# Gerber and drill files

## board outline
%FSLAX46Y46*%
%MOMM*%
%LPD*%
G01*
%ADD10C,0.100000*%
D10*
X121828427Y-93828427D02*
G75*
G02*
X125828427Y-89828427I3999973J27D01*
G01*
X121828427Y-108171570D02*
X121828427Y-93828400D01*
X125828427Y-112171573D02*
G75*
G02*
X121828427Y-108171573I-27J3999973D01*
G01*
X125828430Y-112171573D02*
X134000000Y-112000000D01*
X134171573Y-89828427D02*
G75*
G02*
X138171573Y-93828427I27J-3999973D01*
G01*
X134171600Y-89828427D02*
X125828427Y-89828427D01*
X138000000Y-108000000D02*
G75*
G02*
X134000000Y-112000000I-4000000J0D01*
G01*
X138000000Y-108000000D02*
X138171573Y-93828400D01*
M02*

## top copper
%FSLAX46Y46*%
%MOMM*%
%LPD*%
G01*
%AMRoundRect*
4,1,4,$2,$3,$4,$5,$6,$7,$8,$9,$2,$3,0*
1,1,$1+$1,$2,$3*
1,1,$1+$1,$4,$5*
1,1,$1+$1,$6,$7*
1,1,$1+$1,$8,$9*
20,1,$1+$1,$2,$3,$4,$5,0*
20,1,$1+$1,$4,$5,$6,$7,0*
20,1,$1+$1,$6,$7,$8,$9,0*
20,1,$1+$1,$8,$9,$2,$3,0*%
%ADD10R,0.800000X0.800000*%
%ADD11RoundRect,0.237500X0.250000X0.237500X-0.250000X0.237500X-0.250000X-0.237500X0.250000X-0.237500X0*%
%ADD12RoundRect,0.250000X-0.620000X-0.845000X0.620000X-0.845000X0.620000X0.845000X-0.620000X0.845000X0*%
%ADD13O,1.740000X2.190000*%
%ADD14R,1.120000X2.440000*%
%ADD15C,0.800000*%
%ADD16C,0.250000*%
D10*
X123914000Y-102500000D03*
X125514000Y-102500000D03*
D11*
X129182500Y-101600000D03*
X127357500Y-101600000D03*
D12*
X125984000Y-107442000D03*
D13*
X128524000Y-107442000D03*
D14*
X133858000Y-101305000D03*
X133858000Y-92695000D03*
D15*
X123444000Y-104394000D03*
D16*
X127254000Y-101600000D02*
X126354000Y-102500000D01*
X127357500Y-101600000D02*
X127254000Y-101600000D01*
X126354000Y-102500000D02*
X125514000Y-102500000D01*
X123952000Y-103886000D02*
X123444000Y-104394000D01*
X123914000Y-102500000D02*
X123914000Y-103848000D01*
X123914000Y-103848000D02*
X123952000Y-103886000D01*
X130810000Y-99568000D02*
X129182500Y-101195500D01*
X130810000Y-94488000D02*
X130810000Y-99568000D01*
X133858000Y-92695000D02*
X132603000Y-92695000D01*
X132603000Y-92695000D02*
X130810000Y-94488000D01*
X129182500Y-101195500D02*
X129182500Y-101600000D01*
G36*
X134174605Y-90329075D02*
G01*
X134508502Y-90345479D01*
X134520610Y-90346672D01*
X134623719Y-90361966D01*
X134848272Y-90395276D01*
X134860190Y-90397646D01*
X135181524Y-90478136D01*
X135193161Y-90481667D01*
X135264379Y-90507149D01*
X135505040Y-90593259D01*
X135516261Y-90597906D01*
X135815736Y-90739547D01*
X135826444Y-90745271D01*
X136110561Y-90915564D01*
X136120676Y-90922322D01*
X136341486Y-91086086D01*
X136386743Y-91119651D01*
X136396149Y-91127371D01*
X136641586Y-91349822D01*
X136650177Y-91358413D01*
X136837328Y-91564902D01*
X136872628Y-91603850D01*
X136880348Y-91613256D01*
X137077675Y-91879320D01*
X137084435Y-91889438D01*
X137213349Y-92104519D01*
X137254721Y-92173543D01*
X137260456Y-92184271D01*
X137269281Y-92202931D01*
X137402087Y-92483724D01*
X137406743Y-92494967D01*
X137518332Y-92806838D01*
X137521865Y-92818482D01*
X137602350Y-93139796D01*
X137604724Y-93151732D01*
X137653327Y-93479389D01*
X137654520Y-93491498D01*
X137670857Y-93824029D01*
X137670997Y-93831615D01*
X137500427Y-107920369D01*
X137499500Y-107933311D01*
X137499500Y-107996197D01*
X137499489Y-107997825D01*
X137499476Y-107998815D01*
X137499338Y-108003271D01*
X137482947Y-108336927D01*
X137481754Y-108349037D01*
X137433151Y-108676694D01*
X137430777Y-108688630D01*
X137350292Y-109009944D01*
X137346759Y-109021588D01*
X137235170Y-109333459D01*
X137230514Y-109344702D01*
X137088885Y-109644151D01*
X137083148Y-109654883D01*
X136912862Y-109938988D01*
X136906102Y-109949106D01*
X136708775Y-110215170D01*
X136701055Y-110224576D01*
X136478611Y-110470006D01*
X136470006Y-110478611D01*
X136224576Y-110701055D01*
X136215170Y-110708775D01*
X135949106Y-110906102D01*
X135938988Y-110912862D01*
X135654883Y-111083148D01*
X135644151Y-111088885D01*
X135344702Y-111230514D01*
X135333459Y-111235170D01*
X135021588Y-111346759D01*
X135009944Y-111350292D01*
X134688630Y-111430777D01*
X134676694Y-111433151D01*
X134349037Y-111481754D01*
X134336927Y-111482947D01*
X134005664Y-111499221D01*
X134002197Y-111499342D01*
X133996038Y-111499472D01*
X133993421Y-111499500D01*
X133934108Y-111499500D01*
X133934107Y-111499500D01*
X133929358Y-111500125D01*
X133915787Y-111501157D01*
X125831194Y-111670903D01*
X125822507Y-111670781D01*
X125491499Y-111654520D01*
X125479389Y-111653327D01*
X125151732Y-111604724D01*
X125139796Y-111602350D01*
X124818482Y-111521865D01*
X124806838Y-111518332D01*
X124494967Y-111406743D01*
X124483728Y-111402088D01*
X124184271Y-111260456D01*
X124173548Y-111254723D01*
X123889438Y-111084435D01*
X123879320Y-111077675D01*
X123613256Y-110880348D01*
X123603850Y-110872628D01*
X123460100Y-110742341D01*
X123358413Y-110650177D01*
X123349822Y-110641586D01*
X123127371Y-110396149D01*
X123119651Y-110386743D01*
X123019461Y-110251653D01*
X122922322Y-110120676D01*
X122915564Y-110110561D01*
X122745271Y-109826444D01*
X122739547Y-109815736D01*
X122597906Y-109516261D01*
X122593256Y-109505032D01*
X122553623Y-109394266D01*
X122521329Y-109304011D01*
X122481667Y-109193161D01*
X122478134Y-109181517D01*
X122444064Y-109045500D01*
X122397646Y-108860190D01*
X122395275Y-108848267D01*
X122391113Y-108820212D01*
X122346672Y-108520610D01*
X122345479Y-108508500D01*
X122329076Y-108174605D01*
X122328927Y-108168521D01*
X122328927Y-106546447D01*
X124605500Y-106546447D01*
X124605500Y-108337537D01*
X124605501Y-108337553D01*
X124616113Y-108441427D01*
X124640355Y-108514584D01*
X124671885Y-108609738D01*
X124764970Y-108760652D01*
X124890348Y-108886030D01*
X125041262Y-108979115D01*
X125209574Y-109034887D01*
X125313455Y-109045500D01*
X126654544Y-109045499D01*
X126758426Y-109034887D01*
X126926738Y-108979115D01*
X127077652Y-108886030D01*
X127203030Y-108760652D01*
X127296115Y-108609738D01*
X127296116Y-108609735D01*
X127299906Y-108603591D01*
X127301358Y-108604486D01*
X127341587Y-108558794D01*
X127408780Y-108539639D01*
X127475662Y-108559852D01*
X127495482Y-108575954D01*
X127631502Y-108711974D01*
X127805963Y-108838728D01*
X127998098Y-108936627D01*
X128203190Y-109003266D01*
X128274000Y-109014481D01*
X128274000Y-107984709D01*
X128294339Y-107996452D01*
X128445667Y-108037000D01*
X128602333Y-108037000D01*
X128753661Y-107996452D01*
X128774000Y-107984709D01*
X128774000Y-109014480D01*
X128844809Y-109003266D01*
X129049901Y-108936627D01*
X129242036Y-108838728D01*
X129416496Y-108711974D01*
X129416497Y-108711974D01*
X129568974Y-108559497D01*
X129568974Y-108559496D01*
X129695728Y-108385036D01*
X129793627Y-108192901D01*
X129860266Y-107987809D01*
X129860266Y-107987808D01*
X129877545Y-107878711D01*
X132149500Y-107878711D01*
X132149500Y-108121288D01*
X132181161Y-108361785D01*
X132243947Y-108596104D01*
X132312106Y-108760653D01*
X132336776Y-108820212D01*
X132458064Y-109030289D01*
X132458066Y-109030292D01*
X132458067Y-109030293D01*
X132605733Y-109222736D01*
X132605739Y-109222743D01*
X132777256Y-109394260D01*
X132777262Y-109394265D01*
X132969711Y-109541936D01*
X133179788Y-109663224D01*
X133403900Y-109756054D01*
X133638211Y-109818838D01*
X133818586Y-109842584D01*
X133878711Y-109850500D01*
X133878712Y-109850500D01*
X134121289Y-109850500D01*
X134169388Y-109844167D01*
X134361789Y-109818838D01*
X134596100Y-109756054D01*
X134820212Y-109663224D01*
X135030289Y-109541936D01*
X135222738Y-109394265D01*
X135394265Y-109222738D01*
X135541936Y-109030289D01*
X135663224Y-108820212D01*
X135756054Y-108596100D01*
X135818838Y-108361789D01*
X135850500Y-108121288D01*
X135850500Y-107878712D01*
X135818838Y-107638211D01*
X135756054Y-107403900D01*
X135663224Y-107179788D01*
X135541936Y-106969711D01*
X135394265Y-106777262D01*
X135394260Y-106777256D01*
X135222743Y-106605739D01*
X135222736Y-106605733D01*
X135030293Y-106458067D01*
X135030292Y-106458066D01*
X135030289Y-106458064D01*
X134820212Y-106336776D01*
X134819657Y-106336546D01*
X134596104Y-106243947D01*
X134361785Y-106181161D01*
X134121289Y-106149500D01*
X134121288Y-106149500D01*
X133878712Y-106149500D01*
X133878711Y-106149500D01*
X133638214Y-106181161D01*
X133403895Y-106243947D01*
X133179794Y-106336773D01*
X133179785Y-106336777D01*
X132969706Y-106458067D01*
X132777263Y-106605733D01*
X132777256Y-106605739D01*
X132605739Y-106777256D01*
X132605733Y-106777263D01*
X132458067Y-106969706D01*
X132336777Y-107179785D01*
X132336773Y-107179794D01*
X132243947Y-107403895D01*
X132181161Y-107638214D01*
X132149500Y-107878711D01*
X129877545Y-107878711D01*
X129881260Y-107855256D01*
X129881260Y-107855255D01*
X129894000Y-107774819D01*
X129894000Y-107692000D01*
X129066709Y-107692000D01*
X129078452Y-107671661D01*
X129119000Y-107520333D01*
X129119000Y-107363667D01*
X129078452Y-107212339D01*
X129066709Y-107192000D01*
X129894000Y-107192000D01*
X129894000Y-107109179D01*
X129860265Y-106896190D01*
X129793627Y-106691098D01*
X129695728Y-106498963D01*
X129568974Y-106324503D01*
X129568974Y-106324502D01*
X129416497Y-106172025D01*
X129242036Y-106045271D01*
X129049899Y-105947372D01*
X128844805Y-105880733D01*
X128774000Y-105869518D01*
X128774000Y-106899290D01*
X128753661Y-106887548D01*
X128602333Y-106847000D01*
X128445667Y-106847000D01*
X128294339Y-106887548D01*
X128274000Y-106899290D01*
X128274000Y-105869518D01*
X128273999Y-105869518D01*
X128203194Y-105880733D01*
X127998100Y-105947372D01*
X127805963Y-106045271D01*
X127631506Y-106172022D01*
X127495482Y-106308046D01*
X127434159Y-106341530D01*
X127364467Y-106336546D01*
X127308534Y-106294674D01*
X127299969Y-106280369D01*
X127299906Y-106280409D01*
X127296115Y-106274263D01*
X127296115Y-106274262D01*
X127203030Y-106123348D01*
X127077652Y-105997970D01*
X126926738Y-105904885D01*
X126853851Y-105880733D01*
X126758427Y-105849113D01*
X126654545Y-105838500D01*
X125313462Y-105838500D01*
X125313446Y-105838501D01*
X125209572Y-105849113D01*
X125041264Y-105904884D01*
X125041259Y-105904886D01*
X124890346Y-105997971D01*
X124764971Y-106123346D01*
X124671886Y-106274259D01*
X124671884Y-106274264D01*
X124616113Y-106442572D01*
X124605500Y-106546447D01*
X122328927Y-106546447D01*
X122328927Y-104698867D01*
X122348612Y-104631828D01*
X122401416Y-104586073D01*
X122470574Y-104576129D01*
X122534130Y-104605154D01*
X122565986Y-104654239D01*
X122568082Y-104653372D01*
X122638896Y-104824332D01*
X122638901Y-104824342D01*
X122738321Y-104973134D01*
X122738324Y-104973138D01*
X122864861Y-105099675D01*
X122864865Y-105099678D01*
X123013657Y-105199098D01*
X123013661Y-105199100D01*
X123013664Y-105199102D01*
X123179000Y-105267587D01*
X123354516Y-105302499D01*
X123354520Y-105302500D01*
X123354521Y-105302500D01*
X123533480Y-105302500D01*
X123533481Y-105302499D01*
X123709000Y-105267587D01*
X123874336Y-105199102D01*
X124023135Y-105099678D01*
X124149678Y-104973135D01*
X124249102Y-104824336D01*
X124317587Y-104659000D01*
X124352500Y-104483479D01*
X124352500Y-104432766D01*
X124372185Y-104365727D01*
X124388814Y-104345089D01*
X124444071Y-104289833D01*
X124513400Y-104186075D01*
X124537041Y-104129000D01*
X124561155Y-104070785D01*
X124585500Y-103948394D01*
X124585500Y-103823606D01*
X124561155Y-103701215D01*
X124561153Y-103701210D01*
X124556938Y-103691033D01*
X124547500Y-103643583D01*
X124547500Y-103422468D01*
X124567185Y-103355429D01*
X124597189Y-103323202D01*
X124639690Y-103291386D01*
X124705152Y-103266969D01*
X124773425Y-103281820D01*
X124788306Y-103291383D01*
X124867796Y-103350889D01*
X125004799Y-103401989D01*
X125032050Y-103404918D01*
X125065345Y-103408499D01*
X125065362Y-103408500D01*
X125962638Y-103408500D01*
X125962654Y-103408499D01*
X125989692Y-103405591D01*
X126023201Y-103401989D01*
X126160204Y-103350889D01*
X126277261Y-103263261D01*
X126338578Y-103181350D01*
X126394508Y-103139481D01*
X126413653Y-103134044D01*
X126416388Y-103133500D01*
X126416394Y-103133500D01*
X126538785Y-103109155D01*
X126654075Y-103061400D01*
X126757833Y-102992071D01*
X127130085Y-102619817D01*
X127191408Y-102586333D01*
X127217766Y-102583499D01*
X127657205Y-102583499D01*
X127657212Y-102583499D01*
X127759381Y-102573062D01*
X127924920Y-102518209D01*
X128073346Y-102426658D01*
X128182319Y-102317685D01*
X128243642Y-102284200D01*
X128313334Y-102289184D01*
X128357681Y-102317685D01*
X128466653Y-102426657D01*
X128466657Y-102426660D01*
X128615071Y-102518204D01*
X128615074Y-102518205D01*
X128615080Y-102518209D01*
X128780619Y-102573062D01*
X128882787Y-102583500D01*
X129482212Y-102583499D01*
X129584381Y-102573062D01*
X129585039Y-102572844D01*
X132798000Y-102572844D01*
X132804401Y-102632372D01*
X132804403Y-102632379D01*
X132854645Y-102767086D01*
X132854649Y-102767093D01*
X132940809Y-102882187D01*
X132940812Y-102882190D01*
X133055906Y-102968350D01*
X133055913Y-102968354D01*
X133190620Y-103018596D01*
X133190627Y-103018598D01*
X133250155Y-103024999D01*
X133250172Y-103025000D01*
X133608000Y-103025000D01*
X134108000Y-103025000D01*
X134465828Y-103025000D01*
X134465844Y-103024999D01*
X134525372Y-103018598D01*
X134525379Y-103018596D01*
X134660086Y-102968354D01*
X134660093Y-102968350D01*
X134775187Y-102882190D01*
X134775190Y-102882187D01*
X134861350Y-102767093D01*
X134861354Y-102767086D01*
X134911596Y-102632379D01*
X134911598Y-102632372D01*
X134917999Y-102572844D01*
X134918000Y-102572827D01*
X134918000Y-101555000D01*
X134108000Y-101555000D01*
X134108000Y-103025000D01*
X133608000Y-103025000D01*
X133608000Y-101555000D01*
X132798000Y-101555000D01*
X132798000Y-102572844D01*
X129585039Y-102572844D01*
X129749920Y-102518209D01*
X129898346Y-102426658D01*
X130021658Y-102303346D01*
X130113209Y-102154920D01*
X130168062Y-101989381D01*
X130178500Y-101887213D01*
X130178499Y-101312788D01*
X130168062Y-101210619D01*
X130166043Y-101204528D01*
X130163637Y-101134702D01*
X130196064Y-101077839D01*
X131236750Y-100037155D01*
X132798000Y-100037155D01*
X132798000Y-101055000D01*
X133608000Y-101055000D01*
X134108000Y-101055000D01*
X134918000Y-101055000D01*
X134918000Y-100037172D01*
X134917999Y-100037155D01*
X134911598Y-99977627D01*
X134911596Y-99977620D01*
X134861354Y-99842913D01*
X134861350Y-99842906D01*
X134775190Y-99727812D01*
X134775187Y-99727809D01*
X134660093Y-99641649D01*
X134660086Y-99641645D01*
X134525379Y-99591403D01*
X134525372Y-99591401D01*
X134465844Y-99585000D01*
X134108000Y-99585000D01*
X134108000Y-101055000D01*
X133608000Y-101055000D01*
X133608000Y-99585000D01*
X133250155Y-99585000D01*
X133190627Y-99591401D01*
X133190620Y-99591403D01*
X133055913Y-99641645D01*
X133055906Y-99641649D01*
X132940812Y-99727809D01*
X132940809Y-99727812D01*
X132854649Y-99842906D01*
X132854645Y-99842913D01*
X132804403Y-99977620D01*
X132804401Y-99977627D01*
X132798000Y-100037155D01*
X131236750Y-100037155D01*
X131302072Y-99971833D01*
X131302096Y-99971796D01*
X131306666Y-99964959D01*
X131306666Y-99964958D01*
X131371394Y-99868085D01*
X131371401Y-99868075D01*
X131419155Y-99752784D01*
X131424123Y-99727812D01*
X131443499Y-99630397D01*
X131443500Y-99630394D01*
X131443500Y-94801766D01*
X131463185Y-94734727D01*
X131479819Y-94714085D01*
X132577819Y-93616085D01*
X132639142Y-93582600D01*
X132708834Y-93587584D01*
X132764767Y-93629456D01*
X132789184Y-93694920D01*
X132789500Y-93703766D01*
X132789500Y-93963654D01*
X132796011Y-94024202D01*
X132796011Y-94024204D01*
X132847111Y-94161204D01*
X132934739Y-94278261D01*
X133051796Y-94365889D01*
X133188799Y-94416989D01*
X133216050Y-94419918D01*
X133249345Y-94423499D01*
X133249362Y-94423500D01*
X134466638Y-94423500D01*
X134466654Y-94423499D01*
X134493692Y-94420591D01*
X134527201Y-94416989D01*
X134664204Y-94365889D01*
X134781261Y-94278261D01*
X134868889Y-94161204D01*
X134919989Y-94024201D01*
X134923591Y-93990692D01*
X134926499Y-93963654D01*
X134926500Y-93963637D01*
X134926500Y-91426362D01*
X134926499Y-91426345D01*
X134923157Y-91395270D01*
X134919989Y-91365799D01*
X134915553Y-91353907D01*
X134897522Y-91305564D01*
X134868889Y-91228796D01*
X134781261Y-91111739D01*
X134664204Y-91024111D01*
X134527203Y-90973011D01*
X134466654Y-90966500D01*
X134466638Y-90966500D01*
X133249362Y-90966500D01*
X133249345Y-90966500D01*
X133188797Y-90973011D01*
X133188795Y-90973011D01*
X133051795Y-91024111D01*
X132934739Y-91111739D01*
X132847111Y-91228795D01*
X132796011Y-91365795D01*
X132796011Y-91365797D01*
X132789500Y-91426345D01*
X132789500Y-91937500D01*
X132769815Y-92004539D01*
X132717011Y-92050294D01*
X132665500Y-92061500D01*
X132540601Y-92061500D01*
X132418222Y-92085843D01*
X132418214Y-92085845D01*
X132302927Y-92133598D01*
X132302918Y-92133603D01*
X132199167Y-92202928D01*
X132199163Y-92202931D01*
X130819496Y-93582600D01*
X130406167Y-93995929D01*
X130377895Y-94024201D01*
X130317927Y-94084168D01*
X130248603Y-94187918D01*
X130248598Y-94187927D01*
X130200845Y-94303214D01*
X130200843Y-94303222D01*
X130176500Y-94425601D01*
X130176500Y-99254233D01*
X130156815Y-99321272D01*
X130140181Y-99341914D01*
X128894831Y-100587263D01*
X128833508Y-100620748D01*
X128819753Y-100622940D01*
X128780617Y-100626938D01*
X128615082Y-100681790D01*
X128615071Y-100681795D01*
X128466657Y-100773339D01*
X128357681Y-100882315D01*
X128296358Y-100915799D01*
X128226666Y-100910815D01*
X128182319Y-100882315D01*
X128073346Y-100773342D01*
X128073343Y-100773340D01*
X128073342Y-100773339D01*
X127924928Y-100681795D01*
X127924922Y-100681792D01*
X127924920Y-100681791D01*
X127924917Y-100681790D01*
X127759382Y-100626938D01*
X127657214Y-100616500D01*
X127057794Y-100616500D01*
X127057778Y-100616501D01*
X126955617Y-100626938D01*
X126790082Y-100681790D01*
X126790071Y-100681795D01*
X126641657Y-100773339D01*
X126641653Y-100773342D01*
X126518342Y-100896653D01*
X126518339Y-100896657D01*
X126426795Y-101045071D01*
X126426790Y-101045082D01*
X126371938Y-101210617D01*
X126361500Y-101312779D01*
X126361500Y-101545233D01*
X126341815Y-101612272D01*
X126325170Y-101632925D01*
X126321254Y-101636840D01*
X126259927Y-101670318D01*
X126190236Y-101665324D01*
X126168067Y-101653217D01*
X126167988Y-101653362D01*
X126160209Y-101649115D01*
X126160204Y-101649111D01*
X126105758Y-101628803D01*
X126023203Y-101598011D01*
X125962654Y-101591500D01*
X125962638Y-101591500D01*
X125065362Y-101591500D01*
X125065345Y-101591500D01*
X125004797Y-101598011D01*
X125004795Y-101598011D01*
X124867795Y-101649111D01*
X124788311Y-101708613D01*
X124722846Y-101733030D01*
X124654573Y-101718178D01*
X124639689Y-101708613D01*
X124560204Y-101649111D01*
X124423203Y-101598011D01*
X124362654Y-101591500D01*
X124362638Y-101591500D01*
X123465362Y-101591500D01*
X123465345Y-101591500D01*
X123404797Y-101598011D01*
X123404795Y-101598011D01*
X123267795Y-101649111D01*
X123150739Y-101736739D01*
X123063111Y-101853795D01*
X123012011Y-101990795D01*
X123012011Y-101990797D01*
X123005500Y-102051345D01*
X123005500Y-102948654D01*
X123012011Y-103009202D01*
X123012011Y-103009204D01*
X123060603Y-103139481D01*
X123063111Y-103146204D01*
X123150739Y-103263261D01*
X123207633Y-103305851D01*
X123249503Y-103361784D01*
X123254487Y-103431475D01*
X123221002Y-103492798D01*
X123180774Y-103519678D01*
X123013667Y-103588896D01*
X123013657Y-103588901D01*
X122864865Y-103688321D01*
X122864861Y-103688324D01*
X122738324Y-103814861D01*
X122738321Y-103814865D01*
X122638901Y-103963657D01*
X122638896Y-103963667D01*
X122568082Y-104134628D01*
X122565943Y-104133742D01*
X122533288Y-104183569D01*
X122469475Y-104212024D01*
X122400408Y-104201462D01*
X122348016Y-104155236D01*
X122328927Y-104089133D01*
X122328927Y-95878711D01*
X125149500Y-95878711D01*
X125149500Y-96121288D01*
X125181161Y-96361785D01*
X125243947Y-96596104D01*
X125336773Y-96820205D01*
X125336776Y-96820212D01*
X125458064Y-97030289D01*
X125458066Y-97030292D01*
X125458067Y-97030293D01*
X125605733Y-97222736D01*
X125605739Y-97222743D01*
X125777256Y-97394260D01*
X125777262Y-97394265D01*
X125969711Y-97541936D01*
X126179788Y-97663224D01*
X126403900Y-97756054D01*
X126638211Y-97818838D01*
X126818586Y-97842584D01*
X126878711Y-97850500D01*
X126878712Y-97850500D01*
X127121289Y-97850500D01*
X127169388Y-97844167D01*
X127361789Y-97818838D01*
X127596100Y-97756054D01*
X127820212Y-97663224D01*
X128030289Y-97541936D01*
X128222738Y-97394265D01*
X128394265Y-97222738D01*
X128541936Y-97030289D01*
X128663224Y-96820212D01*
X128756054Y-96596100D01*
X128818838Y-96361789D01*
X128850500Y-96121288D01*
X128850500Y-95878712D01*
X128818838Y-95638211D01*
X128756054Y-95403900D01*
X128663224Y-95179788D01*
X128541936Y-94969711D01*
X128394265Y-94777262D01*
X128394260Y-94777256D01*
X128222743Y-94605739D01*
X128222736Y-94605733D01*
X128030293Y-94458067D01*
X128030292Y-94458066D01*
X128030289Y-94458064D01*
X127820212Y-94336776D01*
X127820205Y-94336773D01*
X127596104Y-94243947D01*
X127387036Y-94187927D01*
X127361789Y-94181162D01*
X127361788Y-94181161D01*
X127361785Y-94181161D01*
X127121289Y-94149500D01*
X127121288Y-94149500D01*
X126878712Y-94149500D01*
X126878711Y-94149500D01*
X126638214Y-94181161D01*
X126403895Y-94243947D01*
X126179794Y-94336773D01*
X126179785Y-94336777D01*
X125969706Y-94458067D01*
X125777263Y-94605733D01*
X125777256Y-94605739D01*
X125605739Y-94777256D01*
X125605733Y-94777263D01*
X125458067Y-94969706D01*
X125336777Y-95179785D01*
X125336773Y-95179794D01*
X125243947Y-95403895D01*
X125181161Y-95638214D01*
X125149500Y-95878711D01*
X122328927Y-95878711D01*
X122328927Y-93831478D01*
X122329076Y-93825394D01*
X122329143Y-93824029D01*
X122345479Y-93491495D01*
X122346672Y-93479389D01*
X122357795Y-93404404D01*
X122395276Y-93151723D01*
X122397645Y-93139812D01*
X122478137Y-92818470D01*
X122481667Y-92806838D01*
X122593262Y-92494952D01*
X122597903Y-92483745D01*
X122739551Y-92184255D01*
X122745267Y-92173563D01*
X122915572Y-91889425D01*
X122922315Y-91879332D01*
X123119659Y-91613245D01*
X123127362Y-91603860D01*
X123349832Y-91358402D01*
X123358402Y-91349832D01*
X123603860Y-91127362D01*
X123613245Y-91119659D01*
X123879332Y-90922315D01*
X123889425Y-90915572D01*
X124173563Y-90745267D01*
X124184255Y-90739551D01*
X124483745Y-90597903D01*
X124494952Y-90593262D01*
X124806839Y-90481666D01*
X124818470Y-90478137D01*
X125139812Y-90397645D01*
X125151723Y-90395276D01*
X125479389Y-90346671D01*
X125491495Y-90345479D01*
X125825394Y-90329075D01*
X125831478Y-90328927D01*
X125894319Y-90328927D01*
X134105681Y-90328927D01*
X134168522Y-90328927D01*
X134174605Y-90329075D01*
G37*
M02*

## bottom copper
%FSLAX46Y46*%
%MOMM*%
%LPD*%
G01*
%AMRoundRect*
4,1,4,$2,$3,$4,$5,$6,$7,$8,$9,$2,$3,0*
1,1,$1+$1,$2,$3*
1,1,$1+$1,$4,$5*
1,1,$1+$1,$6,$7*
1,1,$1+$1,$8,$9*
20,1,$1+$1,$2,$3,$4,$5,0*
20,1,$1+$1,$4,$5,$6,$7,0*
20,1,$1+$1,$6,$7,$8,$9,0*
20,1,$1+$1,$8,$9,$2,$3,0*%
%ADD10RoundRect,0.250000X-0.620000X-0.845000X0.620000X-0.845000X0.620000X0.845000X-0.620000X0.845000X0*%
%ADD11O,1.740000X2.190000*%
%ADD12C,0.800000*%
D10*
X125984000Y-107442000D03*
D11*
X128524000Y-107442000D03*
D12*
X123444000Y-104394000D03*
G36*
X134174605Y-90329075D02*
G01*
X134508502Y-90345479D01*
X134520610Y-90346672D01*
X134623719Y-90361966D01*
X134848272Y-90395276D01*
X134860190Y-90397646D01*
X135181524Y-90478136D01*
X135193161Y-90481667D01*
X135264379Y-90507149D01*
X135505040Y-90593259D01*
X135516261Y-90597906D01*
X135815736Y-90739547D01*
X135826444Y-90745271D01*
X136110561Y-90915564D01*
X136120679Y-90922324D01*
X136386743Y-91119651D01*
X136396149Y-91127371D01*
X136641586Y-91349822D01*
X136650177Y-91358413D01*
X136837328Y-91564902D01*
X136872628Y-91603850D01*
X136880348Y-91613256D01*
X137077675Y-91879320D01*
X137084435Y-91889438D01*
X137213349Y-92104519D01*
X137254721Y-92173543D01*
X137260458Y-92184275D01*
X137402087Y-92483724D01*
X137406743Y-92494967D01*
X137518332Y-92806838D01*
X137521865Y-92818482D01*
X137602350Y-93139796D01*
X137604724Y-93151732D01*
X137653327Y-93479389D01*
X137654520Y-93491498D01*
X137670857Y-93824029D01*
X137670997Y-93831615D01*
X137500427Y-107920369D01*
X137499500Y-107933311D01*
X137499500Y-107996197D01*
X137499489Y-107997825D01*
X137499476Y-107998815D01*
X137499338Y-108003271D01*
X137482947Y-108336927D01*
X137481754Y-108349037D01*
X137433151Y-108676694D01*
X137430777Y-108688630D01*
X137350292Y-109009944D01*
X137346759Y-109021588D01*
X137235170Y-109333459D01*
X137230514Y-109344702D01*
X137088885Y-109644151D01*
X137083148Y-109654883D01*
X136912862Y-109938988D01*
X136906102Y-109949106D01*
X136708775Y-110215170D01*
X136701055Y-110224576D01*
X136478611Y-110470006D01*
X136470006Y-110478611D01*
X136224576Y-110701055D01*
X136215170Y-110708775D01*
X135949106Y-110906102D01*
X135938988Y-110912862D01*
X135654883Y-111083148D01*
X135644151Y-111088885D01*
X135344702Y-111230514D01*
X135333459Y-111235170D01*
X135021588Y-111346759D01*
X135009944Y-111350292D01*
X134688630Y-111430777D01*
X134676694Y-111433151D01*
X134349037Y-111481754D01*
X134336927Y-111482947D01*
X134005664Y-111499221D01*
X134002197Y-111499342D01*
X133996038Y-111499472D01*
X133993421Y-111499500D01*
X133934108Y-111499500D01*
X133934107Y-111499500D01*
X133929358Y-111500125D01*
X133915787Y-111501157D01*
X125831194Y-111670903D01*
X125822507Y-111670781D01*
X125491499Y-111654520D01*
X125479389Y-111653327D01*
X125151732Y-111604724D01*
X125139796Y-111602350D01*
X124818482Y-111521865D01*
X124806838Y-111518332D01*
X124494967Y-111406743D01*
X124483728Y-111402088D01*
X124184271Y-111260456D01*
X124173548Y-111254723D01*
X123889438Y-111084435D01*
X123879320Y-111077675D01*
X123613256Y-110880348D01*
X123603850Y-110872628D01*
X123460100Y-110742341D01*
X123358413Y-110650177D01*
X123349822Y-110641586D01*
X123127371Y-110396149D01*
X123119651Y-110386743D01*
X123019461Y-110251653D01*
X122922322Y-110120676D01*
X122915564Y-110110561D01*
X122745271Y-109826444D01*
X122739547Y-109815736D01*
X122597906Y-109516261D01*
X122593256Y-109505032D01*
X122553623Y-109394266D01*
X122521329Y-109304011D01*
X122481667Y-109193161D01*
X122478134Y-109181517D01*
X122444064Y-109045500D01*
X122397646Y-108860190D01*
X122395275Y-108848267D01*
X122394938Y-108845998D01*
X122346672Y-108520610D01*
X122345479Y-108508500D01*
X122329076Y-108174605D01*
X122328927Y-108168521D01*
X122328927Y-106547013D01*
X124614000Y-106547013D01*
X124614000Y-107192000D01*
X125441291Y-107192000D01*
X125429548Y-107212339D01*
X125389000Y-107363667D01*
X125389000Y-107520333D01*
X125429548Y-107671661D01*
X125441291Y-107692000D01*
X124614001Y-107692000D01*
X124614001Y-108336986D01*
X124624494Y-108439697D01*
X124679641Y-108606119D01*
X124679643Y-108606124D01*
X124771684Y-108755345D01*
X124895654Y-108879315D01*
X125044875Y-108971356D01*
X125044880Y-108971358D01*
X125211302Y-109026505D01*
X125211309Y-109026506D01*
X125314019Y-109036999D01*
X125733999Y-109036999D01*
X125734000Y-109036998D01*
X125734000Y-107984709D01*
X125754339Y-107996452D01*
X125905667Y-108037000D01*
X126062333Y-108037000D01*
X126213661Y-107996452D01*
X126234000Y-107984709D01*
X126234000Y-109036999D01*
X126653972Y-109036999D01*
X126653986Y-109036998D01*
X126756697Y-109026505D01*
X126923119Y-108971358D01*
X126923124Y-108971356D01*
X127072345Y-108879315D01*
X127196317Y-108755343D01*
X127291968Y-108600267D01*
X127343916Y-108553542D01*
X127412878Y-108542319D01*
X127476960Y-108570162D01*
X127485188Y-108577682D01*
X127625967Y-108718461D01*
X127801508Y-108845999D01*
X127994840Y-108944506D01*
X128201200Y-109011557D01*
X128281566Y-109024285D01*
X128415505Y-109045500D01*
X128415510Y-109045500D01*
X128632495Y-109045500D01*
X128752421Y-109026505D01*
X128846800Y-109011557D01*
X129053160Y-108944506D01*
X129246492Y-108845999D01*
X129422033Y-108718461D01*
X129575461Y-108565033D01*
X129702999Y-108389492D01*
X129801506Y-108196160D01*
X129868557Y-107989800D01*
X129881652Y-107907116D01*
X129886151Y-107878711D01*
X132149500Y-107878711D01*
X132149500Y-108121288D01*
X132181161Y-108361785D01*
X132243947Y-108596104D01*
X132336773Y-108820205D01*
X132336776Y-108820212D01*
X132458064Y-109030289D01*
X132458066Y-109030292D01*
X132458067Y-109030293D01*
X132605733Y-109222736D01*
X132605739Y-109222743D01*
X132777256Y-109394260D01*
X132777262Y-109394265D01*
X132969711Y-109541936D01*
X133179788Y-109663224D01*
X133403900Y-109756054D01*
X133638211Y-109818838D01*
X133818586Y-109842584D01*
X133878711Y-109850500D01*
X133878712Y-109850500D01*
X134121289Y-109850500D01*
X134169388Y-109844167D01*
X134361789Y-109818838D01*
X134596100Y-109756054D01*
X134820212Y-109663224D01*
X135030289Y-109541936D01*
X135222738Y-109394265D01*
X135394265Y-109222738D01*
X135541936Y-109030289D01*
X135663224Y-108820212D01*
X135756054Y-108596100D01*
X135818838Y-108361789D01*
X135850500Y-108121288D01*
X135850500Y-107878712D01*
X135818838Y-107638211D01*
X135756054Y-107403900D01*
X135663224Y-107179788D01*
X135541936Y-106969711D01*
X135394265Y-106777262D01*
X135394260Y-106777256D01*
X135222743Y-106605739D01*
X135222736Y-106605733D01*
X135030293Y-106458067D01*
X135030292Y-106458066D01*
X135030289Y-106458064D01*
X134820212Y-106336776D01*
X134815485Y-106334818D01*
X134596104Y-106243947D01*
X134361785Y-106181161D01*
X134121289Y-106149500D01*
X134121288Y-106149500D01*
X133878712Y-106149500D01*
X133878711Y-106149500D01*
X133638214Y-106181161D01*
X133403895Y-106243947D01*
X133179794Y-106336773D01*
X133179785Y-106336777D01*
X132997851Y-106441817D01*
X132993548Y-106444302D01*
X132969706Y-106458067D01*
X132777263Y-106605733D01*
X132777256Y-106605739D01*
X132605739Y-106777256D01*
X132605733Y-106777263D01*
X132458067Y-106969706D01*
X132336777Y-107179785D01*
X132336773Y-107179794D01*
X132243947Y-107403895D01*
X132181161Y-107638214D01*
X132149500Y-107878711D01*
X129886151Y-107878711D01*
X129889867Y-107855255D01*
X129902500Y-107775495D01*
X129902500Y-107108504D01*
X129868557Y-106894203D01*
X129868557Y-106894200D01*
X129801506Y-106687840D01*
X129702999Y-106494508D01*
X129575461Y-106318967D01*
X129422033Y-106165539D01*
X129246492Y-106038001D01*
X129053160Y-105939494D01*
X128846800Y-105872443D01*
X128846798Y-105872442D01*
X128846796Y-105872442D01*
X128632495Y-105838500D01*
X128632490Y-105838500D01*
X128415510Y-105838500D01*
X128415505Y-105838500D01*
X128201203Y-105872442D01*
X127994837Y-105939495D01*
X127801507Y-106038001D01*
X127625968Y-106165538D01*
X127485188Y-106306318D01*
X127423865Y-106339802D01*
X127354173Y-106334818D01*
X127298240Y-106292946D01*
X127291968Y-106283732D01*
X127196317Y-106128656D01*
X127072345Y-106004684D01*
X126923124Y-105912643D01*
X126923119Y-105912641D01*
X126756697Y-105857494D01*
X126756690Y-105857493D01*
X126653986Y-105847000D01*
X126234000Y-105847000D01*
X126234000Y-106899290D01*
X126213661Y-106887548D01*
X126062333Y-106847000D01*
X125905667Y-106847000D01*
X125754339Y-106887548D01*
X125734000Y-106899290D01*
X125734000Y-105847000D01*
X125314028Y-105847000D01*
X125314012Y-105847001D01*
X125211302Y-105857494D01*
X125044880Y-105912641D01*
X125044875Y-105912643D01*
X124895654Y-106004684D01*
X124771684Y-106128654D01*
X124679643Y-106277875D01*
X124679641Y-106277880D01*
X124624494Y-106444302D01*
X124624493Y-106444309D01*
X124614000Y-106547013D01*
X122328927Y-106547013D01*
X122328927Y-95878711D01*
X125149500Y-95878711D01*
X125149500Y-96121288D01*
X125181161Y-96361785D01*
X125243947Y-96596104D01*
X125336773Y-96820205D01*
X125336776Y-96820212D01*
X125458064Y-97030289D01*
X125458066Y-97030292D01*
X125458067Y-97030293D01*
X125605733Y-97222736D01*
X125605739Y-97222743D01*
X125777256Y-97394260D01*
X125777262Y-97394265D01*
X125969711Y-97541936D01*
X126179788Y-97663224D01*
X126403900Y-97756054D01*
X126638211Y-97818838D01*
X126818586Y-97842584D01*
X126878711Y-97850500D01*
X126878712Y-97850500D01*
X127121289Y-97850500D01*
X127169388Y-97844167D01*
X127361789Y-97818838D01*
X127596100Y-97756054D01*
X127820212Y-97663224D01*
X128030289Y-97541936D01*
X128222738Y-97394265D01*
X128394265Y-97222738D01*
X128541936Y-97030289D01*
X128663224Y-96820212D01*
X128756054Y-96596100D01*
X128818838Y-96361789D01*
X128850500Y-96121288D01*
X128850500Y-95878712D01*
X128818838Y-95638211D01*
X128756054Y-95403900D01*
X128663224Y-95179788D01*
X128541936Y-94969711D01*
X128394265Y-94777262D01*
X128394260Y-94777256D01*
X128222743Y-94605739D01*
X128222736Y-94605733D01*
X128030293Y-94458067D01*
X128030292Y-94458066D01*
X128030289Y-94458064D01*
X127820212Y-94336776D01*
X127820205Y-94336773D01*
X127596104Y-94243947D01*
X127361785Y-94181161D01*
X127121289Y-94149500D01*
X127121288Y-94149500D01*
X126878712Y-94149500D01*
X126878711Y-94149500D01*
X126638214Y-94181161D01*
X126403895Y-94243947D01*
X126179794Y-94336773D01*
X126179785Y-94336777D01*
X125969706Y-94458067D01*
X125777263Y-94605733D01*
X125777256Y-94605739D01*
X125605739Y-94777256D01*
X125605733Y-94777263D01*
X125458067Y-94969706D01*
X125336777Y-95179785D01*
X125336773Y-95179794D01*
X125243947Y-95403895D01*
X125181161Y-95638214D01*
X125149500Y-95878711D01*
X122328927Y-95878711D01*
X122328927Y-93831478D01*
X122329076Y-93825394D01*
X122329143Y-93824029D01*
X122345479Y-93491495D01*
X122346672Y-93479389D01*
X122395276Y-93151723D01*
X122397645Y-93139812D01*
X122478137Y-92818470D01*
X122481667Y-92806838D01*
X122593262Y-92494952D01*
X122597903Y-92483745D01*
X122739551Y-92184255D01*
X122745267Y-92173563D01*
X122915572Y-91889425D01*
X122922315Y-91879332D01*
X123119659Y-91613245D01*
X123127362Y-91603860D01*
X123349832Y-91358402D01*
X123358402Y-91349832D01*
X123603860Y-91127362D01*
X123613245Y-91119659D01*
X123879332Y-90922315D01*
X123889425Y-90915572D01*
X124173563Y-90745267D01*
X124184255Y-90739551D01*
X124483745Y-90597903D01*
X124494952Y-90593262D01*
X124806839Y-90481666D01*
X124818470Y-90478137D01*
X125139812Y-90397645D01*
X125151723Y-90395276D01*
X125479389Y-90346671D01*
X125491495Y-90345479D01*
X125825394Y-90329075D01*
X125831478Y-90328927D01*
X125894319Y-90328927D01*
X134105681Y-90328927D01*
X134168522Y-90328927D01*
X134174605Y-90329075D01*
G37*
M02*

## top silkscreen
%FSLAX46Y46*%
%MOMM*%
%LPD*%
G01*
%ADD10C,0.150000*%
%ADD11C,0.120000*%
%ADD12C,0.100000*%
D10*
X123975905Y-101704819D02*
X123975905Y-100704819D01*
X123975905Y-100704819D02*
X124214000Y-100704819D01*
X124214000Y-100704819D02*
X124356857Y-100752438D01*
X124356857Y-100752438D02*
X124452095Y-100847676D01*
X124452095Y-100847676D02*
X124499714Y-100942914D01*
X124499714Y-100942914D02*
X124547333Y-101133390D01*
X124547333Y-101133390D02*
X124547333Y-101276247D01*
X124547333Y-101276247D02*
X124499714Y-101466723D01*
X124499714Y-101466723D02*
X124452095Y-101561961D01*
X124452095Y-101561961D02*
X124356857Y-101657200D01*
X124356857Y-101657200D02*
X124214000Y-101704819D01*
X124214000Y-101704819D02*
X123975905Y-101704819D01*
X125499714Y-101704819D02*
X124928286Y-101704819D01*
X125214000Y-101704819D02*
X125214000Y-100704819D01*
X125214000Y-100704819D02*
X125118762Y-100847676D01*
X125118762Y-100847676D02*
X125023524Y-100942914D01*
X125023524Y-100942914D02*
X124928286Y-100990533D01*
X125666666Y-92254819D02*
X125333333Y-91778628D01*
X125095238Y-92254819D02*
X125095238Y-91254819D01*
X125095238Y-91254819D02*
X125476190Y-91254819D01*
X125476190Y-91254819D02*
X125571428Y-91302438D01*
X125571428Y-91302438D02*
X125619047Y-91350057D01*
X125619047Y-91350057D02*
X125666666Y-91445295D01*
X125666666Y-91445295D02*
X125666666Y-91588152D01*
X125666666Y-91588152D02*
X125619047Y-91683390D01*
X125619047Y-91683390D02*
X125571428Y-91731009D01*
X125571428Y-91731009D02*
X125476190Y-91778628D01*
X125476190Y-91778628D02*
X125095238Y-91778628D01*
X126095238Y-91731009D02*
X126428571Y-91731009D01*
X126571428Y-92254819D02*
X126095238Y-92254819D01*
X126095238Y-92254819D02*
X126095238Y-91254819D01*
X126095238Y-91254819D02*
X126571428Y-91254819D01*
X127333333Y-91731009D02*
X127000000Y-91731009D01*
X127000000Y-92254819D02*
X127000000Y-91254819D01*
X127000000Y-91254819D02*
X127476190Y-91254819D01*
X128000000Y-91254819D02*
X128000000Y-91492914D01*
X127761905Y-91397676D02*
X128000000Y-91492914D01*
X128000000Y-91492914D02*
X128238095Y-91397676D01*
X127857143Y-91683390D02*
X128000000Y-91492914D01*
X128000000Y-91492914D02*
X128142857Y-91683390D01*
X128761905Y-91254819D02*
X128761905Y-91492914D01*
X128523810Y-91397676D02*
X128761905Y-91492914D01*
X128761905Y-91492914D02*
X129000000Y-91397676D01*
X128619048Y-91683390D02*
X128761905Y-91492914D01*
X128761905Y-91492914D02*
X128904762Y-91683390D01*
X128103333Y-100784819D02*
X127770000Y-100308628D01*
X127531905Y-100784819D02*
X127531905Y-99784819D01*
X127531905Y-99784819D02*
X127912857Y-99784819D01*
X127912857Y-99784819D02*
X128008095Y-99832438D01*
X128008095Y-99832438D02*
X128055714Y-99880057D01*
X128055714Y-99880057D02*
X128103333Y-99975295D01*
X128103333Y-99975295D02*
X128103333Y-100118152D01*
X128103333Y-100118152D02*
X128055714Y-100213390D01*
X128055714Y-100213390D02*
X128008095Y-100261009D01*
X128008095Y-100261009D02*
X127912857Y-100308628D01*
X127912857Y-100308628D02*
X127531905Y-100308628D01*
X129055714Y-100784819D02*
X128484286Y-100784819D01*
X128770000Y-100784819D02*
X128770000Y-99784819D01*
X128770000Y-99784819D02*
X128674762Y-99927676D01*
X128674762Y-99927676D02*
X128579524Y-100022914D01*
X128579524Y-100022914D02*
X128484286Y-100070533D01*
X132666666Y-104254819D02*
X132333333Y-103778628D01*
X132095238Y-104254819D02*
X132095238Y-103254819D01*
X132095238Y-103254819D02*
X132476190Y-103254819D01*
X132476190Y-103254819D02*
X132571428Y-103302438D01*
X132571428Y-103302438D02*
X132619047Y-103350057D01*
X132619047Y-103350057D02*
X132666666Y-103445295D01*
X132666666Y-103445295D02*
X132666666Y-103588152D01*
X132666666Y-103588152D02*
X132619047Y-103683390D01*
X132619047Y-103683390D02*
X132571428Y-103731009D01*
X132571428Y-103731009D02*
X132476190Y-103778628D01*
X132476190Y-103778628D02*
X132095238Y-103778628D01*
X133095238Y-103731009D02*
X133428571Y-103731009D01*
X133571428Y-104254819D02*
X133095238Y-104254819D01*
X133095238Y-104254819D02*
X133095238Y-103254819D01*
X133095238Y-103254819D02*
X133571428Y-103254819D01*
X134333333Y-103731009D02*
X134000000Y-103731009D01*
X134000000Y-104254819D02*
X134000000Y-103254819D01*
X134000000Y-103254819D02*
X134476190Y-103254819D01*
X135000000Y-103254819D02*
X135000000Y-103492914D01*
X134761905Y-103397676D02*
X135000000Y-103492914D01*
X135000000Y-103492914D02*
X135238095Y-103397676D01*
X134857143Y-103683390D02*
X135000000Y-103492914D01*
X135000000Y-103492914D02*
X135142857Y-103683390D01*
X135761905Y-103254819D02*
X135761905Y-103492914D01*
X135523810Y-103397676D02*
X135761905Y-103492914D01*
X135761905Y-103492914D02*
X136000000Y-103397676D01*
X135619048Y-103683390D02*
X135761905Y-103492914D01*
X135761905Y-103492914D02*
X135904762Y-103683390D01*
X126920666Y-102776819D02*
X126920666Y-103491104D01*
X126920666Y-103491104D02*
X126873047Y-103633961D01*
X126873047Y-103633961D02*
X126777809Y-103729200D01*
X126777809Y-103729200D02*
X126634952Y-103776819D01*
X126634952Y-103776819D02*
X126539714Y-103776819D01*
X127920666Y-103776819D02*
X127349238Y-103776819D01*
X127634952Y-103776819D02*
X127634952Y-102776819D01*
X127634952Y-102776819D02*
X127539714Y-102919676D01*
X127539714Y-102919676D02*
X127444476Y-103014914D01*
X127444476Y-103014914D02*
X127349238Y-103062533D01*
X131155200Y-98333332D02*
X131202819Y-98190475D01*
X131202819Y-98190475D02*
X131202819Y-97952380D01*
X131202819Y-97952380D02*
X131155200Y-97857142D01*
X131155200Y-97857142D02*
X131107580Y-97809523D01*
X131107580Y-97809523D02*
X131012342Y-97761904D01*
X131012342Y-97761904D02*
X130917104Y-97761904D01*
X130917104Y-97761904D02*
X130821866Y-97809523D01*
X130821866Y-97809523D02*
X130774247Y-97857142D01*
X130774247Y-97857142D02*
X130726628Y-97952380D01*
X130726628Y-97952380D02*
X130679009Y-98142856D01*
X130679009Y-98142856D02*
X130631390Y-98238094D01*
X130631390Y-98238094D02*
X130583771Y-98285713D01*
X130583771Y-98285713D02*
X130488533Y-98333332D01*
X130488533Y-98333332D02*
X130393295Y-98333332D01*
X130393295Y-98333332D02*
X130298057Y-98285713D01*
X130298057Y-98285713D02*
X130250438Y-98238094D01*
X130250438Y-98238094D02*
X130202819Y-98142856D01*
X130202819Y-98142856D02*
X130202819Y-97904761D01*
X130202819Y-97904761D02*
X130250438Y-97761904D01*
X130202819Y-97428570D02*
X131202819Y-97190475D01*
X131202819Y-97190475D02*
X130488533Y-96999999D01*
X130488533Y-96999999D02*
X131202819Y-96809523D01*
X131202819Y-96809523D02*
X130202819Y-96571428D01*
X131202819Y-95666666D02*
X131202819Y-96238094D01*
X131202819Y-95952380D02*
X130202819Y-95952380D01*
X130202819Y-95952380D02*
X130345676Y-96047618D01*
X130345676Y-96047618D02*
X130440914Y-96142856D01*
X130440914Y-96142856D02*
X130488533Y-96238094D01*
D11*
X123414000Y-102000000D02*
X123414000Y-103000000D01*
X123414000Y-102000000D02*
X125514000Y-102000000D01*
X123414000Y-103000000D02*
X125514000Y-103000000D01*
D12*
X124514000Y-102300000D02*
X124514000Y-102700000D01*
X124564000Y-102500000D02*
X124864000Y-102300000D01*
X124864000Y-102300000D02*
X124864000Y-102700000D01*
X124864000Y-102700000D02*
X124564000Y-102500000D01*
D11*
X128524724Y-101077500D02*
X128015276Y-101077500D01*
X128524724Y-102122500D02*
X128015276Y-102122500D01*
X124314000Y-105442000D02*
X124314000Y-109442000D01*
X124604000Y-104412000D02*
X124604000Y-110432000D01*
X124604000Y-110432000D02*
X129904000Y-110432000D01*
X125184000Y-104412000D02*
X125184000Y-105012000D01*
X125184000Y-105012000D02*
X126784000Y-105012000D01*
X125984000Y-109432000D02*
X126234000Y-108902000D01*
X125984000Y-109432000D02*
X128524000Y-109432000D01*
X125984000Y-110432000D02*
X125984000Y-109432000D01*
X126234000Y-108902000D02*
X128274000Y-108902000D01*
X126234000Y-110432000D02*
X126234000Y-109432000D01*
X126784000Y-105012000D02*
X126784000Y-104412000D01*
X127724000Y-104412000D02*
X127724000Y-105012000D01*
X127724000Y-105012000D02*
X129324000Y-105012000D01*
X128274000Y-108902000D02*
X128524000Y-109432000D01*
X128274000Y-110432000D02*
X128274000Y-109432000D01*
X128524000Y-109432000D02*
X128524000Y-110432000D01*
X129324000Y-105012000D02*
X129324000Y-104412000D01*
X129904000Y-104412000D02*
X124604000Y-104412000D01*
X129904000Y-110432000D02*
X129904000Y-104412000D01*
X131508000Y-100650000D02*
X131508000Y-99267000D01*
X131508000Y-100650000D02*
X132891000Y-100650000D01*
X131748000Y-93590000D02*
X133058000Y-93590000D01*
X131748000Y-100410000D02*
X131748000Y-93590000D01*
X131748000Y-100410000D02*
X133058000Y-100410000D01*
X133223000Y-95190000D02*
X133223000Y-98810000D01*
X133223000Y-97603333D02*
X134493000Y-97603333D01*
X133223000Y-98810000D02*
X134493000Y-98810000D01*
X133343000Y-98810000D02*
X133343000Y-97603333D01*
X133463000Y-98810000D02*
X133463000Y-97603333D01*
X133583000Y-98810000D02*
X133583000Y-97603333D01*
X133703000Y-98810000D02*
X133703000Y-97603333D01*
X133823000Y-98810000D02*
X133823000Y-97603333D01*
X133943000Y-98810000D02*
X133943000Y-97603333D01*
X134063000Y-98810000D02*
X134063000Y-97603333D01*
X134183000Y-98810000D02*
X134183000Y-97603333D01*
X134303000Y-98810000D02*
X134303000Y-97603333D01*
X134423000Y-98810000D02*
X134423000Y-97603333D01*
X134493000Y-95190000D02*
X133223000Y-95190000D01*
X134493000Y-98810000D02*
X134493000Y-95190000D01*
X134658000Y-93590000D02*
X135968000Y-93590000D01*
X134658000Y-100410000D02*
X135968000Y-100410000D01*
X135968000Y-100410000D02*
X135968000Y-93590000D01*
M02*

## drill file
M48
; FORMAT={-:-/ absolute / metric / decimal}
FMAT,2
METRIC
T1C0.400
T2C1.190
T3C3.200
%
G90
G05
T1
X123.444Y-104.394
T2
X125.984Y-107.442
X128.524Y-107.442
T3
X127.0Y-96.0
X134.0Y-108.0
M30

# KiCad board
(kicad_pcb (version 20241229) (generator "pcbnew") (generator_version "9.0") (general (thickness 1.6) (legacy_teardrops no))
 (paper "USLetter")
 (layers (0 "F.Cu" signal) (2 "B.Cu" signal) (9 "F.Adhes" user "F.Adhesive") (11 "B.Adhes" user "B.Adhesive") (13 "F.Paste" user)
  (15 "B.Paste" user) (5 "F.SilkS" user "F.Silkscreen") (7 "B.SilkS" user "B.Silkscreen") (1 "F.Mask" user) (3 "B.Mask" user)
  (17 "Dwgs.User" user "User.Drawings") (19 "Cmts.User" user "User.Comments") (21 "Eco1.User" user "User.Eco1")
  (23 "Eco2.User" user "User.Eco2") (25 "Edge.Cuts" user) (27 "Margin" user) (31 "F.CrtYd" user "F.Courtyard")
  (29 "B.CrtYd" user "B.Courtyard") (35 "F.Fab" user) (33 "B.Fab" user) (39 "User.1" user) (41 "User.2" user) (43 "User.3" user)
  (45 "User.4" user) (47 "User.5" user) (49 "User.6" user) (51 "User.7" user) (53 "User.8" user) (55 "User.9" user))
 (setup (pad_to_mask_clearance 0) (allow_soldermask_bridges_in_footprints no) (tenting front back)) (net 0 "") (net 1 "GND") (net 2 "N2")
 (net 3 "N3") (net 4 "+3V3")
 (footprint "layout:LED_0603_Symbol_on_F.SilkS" (layer "F.Cu") (at 124.714 102.5)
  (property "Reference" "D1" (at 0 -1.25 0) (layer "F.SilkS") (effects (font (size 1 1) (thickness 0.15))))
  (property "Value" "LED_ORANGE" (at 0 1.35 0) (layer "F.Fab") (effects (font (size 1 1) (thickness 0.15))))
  (fp_line (start -1.3 -0.5) (end -1.3 0.5) (stroke (width 0.12) (type solid)) (layer "F.SilkS"))
  (fp_line (start -1.3 -0.5) (end 0.8 -0.5) (stroke (width 0.12) (type solid)) (layer "F.SilkS"))
  (fp_line (start -1.3 0.5) (end 0.8 0.5) (stroke (width 0.12) (type solid)) (layer "F.SilkS"))
  (fp_line (start -0.2 -0.2) (end -0.2 0.2) (stroke (width 0.1) (type solid)) (layer "F.SilkS"))
  (fp_line (start -0.15 0) (end 0.15 -0.2) (stroke (width 0.1) (type solid)) (layer "F.SilkS"))
  (fp_line (start 0.15 -0.2) (end 0.15 0.2) (stroke (width 0.1) (type solid)) (layer "F.SilkS"))
  (fp_line (start 0.15 0.2) (end -0.15 0) (stroke (width 0.1) (type solid)) (layer "F.SilkS"))
  (pad "1" smd rect (at -0.8 0 180) (size 0.8 0.8) (layers "F.Cu" "F.Mask" "F.Paste") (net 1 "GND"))
  (pad "2" smd rect (at 0.8 0 180) (size 0.8 0.8) (layers "F.Cu" "F.Mask" "F.Paste") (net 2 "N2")))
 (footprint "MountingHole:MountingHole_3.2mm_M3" (layer "F.Cu") (at 127 96)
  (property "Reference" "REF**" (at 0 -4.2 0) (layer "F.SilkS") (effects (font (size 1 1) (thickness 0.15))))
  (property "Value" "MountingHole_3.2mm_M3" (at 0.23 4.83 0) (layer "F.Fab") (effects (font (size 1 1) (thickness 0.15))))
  (pad "" np_thru_hole circle (at 0 0) (size 3.2 3.2) (drill 3.2) (layers "*.Cu" "*.Mask")))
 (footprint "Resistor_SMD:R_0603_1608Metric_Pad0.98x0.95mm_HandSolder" (layer "F.Cu") (at 128.27 101.6 180)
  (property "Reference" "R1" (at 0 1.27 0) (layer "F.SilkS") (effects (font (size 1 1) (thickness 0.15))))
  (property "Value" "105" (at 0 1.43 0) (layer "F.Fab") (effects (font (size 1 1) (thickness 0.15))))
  (fp_line (start -0.254724 0.5225) (end 0.254724 0.5225) (stroke (width 0.12) (type solid)) (layer "F.SilkS"))
  (fp_line (start -0.254724 -0.5225) (end 0.254724 -0.5225) (stroke (width 0.12) (type solid)) (layer "F.SilkS"))
  (pad "1" smd roundrect (at -0.9125 0 180) (size 0.975 0.95) (layers "F.Cu" "F.Mask" "F.Paste") (roundrect_rratio 0.25) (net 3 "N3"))
  (pad "2" smd roundrect (at 0.9125 0 180) (size 0.975 0.95) (layers "F.Cu" "F.Mask" "F.Paste") (roundrect_rratio 0.25) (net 2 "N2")))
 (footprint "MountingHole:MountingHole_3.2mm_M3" (layer "F.Cu") (at 134 108)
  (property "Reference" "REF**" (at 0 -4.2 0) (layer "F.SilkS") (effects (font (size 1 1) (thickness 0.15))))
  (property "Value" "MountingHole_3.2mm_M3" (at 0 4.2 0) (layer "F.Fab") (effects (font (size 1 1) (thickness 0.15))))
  (pad "" np_thru_hole circle (at 0 0) (size 3.2 3.2) (drill 3.2) (layers "*.Cu" "*.Mask")))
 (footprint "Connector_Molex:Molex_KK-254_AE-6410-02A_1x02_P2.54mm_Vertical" (layer "F.Cu") (at 125.984 107.442)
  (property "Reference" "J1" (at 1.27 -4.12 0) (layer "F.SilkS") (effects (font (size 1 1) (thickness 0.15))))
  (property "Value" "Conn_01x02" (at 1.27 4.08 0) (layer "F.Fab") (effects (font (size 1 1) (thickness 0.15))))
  (fp_line (start -1.67 -2) (end -1.67 2) (stroke (width 0.12) (type solid)) (layer "F.SilkS"))
  (fp_line (start -1.38 -3.03) (end -1.38 2.99) (stroke (width 0.12) (type solid)) (layer "F.SilkS"))
  (fp_line (start -1.38 2.99) (end 3.92 2.99) (stroke (width 0.12) (type solid)) (layer "F.SilkS"))
  (fp_line (start -0.8 -3.03) (end -0.8 -2.43) (stroke (width 0.12) (type solid)) (layer "F.SilkS"))
  (fp_line (start -0.8 -2.43) (end 0.8 -2.43) (stroke (width 0.12) (type solid)) (layer "F.SilkS"))
  (fp_line (start 0 1.99) (end 0.25 1.46) (stroke (width 0.12) (type solid)) (layer "F.SilkS"))
  (fp_line (start 0 1.99) (end 2.54 1.99) (stroke (width 0.12) (type solid)) (layer "F.SilkS"))
  (fp_line (start 0 2.99) (end 0 1.99) (stroke (width 0.12) (type solid)) (layer "F.SilkS"))
  (fp_line (start 0.25 1.46) (end 2.29 1.46) (stroke (width 0.12) (type solid)) (layer "F.SilkS"))
  (fp_line (start 0.25 2.99) (end 0.25 1.99) (stroke (width 0.12) (type solid)) (layer "F.SilkS"))
  (fp_line (start 0.8 -2.43) (end 0.8 -3.03) (stroke (width 0.12) (type solid)) (layer "F.SilkS"))
  (fp_line (start 1.74 -3.03) (end 1.74 -2.43) (stroke (width 0.12) (type solid)) (layer "F.SilkS"))
  (fp_line (start 1.74 -2.43) (end 3.34 -2.43) (stroke (width 0.12) (type solid)) (layer "F.SilkS"))
  (fp_line (start 2.29 1.46) (end 2.54 1.99) (stroke (width 0.12) (type solid)) (layer "F.SilkS"))
  (fp_line (start 2.29 2.99) (end 2.29 1.99) (stroke (width 0.12) (type solid)) (layer "F.SilkS"))
  (fp_line (start 2.54 1.99) (end 2.54 2.99) (stroke (width 0.12) (type solid)) (layer "F.SilkS"))
  (fp_line (start 3.34 -2.43) (end 3.34 -3.03) (stroke (width 0.12) (type solid)) (layer "F.SilkS"))
  (fp_line (start 3.92 -3.03) (end -1.38 -3.03) (stroke (width 0.12) (type solid)) (layer "F.SilkS"))
  (fp_line (start 3.92 2.99) (end 3.92 -3.03) (stroke (width 0.12) (type solid)) (layer "F.SilkS"))
  (pad "1" thru_hole roundrect (at 0 0) (size 1.74 2.19) (drill 1.19) (layers "*.Cu" "*.Mask") (remove_unused_layers no)
   (roundrect_rratio 0.143678) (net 1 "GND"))
  (pad "2" thru_hole oval (at 2.54 0) (size 1.74 2.19) (drill 1.19) (layers "*.Cu" "*.Mask") (remove_unused_layers no) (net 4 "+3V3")))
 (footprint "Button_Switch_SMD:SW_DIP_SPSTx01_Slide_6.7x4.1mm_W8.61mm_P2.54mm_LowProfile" (layer "F.Cu") (at 133.858 97 90)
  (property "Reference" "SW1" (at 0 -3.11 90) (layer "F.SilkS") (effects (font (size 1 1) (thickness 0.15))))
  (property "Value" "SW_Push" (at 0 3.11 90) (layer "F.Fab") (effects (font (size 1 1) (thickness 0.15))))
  (fp_line (start -3.65 -2.35) (end -2.267 -2.35) (stroke (width 0.12) (type solid)) (layer "F.SilkS"))
  (fp_line (start -3.65 -2.35) (end -3.65 -0.967) (stroke (width 0.12) (type solid)) (layer "F.SilkS"))
  (fp_line (start 3.41 -2.11) (end 3.41 -0.8) (stroke (width 0.12) (type solid)) (layer "F.SilkS"))
  (fp_line (start -3.41 -2.11) (end 3.41 -2.11) (stroke (width 0.12) (type solid)) (layer "F.SilkS"))
  (fp_line (start -3.41 -2.11) (end -3.41 -0.8) (stroke (width 0.12) (type solid)) (layer "F.SilkS"))
  (fp_line (start 1.81 -0.635) (end -1.81 -0.635) (stroke (width 0.12) (type solid)) (layer "F.SilkS"))
  (fp_line (start -0.603333 -0.635) (end -0.603333 0.635) (stroke (width 0.12) (type solid)) (layer "F.SilkS"))
  (fp_line (start -1.81 -0.635) (end -1.81 0.635) (stroke (width 0.12) (type solid)) (layer "F.SilkS"))
  (fp_line (start -1.81 -0.515) (end -0.603333 -0.515) (stroke (width 0.12) (type solid)) (layer "F.SilkS"))
  (fp_line (start -1.81 -0.395) (end -0.603333 -0.395) (stroke (width 0.12) (type solid)) (layer "F.SilkS"))
  (fp_line (start -1.81 -0.275) (end -0.603333 -0.275) (stroke (width 0.12) (type solid)) (layer "F.SilkS"))
  (fp_line (start -1.81 -0.155) (end -0.603333 -0.155) (stroke (width 0.12) (type solid)) (layer "F.SilkS"))
  (fp_line (start -1.81 -0.035) (end -0.603333 -0.035) (stroke (width 0.12) (type solid)) (layer "F.SilkS"))
  (fp_line (start -1.81 0.085) (end -0.603333 0.085) (stroke (width 0.12) (type solid)) (layer "F.SilkS"))
  (fp_line (start -1.81 0.205) (end -0.603333 0.205) (stroke (width 0.12) (type solid)) (layer "F.SilkS"))
  (fp_line (start -1.81 0.325) (end -0.603333 0.325) (stroke (width 0.12) (type solid)) (layer "F.SilkS"))
  (fp_line (start -1.81 0.445) (end -0.603333 0.445) (stroke (width 0.12) (type solid)) (layer "F.SilkS"))
  (fp_line (start -1.81 0.565) (end -0.603333 0.565) (stroke (width 0.12) (type solid)) (layer "F.SilkS"))
  (fp_line (start 1.81 0.635) (end 1.81 -0.635) (stroke (width 0.12) (type solid)) (layer "F.SilkS"))
  (fp_line (start -1.81 0.635) (end 1.81 0.635) (stroke (width 0.12) (type solid)) (layer "F.SilkS"))
  (fp_line (start 3.41 0.8) (end 3.41 2.11) (stroke (width 0.12) (type solid)) (layer "F.SilkS"))
  (fp_line (start -3.41 0.8) (end -3.41 2.11) (stroke (width 0.12) (type solid)) (layer "F.SilkS"))
  (fp_line (start -3.41 2.11) (end 3.41 2.11) (stroke (width 0.12) (type solid)) (layer "F.SilkS"))
  (pad "1" smd rect (at -4.305 0 90) (size 2.44 1.12) (layers "F.Cu" "F.Mask" "F.Paste") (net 4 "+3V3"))
  (pad "2" smd rect (at 4.305 0 90) (size 2.44 1.12) (layers "F.Cu" "F.Mask" "F.Paste") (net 3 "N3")))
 (gr_arc (start 121.828427 93.828427) (mid 123 91) (end 125.828427 89.828427) (stroke (width 0.1) (type default)) (layer "Edge.Cuts"))
 (gr_line (start 121.828427 108.17157) (end 121.828427 93.8284) (stroke (width 0.1) (type default)) (layer "Edge.Cuts"))
 (gr_arc (start 125.828427 112.171573) (mid 123 111) (end 121.828427 108.171573) (stroke (width 0.1) (type default)) (layer "Edge.Cuts"))
 (gr_line (start 125.82843 112.171573) (end 134 112) (stroke (width 0.1) (type default)) (layer "Edge.Cuts"))
 (gr_arc (start 134.171573 89.828427) (mid 137 91) (end 138.171573 93.828427) (stroke (width 0.1) (type default)) (layer "Edge.Cuts"))
 (gr_line (start 134.1716 89.828427) (end 125.828427 89.828427) (stroke (width 0.1) (type default)) (layer "Edge.Cuts"))
 (gr_arc (start 138 108) (mid 136.828427 110.828427) (end 134 112) (stroke (width 0.1) (type default)) (layer "Edge.Cuts"))
 (gr_line (start 138 108) (end 138.171573 93.8284) (stroke (width 0.1) (type default)) (layer "Edge.Cuts"))
 (segment (start 127.254 101.6) (end 126.354 102.5) (width 0.25) (layer "F.Cu") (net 2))
 (segment (start 127.3575 101.6) (end 127.254 101.6) (width 0.25) (layer "F.Cu") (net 2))
 (segment (start 126.354 102.5) (end 125.514 102.5) (width 0.25) (layer "F.Cu") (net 2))
 (segment (start 123.952 103.886) (end 123.444 104.394) (width 0.25) (layer "F.Cu") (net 1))
 (segment (start 123.914 102.5) (end 123.914 103.848) (width 0.25) (layer "F.Cu") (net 1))
 (segment (start 123.914 103.848) (end 123.952 103.886) (width 0.25) (layer "F.Cu") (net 1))
 (via (at 123.444 104.394) (size 0.8) (drill 0.4) (layers "F.Cu" "B.Cu") (free yes) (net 1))
 (segment (start 130.81 99.568) (end 129.1825 101.1955) (width 0.25) (layer "F.Cu") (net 3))
 (segment (start 130.81 94.488) (end 130.81 99.568) (width 0.25) (layer "F.Cu") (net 3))
 (segment (start 133.858 92.695) (end 132.603 92.695) (width 0.25) (layer "F.Cu") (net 3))
 (segment (start 132.603 92.695) (end 130.81 94.488) (width 0.25) (layer "F.Cu") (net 3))
 (segment (start 129.1825 101.1955) (end 129.1825 101.6) (width 0.25) (layer "F.Cu") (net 3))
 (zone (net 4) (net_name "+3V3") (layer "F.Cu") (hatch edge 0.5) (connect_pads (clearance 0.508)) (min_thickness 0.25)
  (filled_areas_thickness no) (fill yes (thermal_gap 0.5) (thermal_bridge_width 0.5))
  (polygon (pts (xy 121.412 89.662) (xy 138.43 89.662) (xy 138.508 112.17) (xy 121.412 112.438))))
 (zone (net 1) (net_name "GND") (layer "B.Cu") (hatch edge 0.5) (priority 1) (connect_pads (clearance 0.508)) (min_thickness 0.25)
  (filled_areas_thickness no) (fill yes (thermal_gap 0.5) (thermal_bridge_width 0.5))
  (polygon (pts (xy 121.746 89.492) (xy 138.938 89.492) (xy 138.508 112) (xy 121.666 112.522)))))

